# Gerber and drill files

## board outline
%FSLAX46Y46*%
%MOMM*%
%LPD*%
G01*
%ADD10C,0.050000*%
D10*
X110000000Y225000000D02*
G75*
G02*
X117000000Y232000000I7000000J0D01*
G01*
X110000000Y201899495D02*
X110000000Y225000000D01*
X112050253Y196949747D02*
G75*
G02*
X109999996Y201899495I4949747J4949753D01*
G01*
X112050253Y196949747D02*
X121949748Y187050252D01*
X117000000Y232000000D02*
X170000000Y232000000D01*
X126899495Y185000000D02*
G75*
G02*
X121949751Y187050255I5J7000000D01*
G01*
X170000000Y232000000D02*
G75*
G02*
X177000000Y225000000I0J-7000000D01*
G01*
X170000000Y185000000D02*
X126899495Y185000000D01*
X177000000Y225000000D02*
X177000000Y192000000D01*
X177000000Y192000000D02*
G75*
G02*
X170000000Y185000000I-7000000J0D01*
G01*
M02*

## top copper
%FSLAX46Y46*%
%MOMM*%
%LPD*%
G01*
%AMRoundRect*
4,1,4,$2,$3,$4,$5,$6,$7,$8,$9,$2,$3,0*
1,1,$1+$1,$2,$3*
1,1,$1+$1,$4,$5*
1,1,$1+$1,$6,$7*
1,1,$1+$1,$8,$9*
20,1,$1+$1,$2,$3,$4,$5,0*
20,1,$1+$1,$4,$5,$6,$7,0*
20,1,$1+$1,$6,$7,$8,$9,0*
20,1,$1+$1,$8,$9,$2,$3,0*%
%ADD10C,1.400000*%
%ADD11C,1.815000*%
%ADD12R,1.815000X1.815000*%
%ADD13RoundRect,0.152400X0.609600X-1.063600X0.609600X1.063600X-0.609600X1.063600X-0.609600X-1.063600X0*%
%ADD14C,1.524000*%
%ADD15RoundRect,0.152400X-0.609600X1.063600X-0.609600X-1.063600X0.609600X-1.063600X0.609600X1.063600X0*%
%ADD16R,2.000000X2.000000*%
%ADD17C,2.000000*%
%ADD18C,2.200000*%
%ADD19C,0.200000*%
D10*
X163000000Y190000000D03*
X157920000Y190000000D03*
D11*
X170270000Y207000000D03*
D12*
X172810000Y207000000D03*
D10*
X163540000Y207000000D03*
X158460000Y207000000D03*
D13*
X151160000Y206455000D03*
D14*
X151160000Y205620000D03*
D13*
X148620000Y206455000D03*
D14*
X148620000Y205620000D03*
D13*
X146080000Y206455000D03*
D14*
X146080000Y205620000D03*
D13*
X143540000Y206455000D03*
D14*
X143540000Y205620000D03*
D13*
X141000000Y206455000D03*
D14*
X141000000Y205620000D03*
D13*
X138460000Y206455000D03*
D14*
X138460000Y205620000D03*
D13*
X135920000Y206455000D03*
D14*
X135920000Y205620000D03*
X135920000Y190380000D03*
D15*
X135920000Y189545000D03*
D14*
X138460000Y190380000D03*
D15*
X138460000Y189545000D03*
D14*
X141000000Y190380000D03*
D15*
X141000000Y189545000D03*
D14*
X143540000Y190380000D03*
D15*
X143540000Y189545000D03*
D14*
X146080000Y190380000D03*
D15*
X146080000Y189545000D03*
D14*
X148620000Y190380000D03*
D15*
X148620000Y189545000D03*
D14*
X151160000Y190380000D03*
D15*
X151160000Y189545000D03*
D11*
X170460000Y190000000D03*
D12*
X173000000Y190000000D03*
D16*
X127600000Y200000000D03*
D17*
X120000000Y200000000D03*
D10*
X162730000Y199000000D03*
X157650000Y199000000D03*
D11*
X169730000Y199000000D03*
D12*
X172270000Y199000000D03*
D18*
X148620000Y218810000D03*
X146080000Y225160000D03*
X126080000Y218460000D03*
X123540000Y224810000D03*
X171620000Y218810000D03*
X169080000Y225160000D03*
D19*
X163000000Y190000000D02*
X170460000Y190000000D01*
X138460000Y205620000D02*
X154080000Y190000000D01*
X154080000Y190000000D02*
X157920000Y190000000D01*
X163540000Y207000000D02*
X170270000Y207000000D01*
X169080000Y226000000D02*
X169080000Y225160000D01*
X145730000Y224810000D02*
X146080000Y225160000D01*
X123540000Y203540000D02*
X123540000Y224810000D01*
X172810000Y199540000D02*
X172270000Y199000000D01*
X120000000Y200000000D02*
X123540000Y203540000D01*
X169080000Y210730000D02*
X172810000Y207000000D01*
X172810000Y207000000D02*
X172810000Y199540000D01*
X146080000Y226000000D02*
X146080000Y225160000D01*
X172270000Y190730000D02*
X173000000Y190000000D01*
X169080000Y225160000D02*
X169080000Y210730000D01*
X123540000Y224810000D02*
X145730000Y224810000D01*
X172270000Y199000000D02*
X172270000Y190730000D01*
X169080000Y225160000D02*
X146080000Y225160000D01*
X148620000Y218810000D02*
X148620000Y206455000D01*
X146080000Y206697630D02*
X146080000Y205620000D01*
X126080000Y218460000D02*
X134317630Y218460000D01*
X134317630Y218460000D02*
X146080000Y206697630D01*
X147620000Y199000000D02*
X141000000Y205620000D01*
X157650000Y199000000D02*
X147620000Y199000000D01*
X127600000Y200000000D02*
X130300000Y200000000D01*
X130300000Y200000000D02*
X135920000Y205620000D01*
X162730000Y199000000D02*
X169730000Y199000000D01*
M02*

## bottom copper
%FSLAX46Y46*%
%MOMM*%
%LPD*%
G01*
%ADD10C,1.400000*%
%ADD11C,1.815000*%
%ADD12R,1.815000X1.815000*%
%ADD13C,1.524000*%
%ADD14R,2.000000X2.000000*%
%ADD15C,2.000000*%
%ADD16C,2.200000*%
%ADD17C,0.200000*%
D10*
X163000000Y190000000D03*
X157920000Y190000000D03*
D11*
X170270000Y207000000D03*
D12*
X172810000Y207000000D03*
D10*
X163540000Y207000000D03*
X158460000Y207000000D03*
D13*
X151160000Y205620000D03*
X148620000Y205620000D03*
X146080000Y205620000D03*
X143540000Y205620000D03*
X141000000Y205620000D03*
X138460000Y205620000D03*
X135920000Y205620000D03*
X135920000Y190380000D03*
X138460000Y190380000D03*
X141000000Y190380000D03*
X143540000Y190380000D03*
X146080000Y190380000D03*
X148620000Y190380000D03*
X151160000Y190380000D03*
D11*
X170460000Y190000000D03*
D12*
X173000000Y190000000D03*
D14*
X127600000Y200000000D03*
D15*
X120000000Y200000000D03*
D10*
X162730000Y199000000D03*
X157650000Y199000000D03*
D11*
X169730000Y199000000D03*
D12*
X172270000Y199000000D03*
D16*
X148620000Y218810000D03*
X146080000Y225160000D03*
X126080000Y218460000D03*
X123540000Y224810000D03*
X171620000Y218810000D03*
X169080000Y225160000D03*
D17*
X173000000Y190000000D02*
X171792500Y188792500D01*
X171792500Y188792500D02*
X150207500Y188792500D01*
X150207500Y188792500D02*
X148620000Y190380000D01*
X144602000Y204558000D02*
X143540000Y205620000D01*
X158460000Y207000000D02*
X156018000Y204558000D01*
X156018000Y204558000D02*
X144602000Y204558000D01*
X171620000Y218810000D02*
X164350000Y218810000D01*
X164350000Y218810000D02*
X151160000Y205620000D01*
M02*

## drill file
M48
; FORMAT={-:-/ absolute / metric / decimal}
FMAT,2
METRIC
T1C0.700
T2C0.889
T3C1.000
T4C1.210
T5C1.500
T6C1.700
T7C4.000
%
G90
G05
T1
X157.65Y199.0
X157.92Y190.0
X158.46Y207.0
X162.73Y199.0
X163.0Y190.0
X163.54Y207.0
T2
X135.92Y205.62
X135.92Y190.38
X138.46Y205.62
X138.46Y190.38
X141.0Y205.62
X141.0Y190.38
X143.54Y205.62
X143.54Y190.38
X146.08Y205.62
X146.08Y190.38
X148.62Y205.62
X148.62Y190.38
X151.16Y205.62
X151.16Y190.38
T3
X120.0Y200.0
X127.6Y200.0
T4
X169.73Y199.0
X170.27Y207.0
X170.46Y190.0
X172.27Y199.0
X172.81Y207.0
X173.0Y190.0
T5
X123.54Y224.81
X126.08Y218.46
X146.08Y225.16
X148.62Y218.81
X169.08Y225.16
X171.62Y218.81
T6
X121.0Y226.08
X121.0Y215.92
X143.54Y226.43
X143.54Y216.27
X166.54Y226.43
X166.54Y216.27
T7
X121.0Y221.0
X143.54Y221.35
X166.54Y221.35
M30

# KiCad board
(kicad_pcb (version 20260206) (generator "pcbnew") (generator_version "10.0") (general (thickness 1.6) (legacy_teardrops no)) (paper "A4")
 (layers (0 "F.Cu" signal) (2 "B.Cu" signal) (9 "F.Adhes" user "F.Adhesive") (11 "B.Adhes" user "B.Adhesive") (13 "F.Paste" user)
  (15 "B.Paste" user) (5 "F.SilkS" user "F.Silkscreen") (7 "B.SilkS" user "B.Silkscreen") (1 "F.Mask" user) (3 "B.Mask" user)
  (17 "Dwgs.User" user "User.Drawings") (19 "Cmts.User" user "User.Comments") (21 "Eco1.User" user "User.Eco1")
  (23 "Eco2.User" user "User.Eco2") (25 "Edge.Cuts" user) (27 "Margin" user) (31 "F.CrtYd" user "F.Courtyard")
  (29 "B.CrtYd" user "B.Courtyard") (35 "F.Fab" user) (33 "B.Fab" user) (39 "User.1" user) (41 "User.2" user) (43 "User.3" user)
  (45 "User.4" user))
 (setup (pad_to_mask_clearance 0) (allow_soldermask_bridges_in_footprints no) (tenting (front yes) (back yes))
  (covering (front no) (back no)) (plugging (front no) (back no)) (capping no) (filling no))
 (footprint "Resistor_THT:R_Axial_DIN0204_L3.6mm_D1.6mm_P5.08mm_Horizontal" (layer "F.Cu") (at 163 -190 180)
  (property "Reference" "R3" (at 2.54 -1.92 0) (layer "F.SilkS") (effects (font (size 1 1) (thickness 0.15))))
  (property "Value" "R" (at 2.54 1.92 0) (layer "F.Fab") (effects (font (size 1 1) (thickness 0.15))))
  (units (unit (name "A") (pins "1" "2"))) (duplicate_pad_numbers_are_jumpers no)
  (pad "1" thru_hole circle (at 0 0 180) (size 1.4 1.4) (drill 0.7) (layers "*.Cu" "*.Mask") (remove_unused_layers no) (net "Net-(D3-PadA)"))
  (pad "2" thru_hole circle (at 5.08 0 180) (size 1.4 1.4) (drill 0.7) (layers "*.Cu" "*.Mask") (remove_unused_layers no) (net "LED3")))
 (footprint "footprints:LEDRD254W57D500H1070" (layer "F.Cu") (at 171.54 -207 180)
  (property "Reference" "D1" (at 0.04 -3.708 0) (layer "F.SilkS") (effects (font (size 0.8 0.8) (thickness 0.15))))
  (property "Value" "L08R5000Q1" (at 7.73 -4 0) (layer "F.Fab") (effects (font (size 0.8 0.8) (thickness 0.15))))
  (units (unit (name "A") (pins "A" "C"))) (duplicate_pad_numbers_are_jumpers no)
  (pad "A" thru_hole circle (at 1.27 0 180) (size 1.815 1.815) (drill 1.21) (layers "*.Cu" "*.Mask") (remove_unused_layers no)
   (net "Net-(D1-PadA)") (solder_mask_margin 0.102))
  (pad "C" thru_hole rect (at -1.27 0 180) (size 1.815 1.815) (drill 1.21) (layers "*.Cu" "*.Mask") (remove_unused_layers no) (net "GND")
   (solder_mask_margin 0.102)))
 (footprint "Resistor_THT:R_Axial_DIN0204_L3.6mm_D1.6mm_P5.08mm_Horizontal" (layer "F.Cu") (at 163.54 -207 180)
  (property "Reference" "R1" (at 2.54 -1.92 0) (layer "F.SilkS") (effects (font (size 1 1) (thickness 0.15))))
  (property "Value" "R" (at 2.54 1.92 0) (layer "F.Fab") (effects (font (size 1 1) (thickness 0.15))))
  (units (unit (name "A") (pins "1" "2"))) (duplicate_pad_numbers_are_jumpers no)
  (pad "1" thru_hole circle (at 0 0 180) (size 1.4 1.4) (drill 0.7) (layers "*.Cu" "*.Mask") (remove_unused_layers no) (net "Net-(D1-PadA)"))
  (pad "2" thru_hole circle (at 5.08 0 180) (size 1.4 1.4) (drill 0.7) (layers "*.Cu" "*.Mask") (remove_unused_layers no) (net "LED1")))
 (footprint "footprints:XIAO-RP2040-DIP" (layer "F.Cu") (at 143.54 -198)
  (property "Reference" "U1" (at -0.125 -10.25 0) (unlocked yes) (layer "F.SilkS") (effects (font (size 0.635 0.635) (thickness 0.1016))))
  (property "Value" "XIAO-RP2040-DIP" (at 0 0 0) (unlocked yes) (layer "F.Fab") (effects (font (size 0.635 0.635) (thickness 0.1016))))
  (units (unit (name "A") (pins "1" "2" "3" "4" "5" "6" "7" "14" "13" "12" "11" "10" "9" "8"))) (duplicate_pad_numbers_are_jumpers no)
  (pad "1" smd roundrect (at 7.62 -8.455 90) (size 2.432 1.524) (layers "F.Cu" "F.Mask") (roundrect_rratio 0.1) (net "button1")
   (thermal_bridge_angle 45))
  (pad "1" thru_hole circle (at 7.62 -7.62 90) (size 1.524 1.524) (drill 0.889) (layers "*.Cu" "*.Mask") (remove_unused_layers no)
   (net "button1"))
  (pad "2" smd roundrect (at 5.08 -8.455 90) (size 2.432 1.524) (layers "F.Cu" "F.Mask") (roundrect_rratio 0.1) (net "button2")
   (thermal_bridge_angle 45))
  (pad "2" thru_hole circle (at 5.08 -7.62 90) (size 1.524 1.524) (drill 0.889) (layers "*.Cu" "*.Mask") (remove_unused_layers no)
   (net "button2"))
  (pad "3" smd roundrect (at 2.54 -8.455 90) (size 2.432 1.524) (layers "F.Cu" "F.Mask") (roundrect_rratio 0.1) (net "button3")
   (thermal_bridge_angle 45))
  (pad "3" thru_hole circle (at 2.54 -7.62 90) (size 1.524 1.524) (drill 0.889) (layers "*.Cu" "*.Mask") (remove_unused_layers no)
   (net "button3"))
  (pad "4" smd roundrect (at 0 -8.455 90) (size 2.432 1.524) (layers "F.Cu" "F.Mask") (roundrect_rratio 0.1) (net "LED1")
   (thermal_bridge_angle 45))
  (pad "4" thru_hole circle (at 0 -7.62 90) (size 1.524 1.524) (drill 0.889) (layers "*.Cu" "*.Mask") (remove_unused_layers no) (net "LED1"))
  (pad "5" smd roundrect (at -2.54 -8.455 90) (size 2.432 1.524) (layers "F.Cu" "F.Mask") (roundrect_rratio 0.1) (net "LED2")
   (thermal_bridge_angle 45))
  (pad "5" thru_hole circle (at -2.54 -7.62 90) (size 1.524 1.524) (drill 0.889) (layers "*.Cu" "*.Mask") (remove_unused_layers no)
   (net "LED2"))
  (pad "6" smd roundrect (at -5.08 -8.455 90) (size 2.432 1.524) (layers "F.Cu" "F.Mask") (roundrect_rratio 0.1) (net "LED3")
   (thermal_bridge_angle 45))
  (pad "6" thru_hole circle (at -5.08 -7.62 90) (size 1.524 1.524) (drill 0.889) (layers "*.Cu" "*.Mask") (remove_unused_layers no)
   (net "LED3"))
  (pad "7" smd roundrect (at -7.62 -8.455 90) (size 2.432 1.524) (layers "F.Cu" "F.Mask") (roundrect_rratio 0.1) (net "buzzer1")
   (thermal_bridge_angle 45))
  (pad "7" thru_hole circle (at -7.62 -7.62 90) (size 1.524 1.524) (drill 0.889) (layers "*.Cu" "*.Mask") (remove_unused_layers no)
   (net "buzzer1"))
  (pad "8" thru_hole circle (at -7.62 7.62 270) (size 1.524 1.524) (drill 0.889) (layers "*.Cu" "*.Mask") (remove_unused_layers no)
   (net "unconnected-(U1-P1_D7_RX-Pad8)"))
  (pad "8" smd roundrect (at -7.62 8.455 270) (size 2.432 1.524) (layers "F.Cu" "F.Mask") (roundrect_rratio 0.1)
   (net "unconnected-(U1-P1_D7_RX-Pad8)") (thermal_bridge_angle 45))
  (pad "9" thru_hole circle (at -5.08 7.62 270) (size 1.524 1.524) (drill 0.889) (layers "*.Cu" "*.Mask") (remove_unused_layers no)
   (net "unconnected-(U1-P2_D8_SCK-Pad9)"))
  (pad "9" smd roundrect (at -5.08 8.455 270) (size 2.432 1.524) (layers "F.Cu" "F.Mask") (roundrect_rratio 0.1)
   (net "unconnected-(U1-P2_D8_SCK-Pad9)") (thermal_bridge_angle 45))
  (pad "10" thru_hole circle (at -2.54 7.62 270) (size 1.524 1.524) (drill 0.889) (layers "*.Cu" "*.Mask") (remove_unused_layers no)
   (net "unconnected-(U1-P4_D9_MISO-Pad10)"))
  (pad "10" smd roundrect (at -2.54 8.455 270) (size 2.432 1.524) (layers "F.Cu" "F.Mask") (roundrect_rratio 0.1)
   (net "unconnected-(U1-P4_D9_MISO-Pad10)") (thermal_bridge_angle 45))
  (pad "11" thru_hole circle (at 0 7.62 270) (size 1.524 1.524) (drill 0.889) (layers "*.Cu" "*.Mask") (remove_unused_layers no)
   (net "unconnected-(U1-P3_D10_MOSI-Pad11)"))
  (pad "11" smd roundrect (at 0 8.455 270) (size 2.432 1.524) (layers "F.Cu" "F.Mask") (roundrect_rratio 0.1)
   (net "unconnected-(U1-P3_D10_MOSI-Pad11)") (thermal_bridge_angle 45))
  (pad "12" thru_hole circle (at 2.54 7.62 270) (size 1.524 1.524) (drill 0.889) (layers "*.Cu" "*.Mask") (remove_unused_layers no)
   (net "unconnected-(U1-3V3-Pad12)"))
  (pad "12" smd roundrect (at 2.54 8.455 270) (size 2.432 1.524) (layers "F.Cu" "F.Mask") (roundrect_rratio 0.1)
   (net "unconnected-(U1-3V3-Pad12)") (thermal_bridge_angle 45))
  (pad "13" thru_hole circle (at 5.08 7.62 270) (size 1.524 1.524) (drill 0.889) (layers "*.Cu" "*.Mask") (remove_unused_layers no)
   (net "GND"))
  (pad "13" smd roundrect (at 5.08 8.455 270) (size 2.432 1.524) (layers "F.Cu" "F.Mask") (roundrect_rratio 0.1) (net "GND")
   (thermal_bridge_angle 45))
  (pad "14" thru_hole circle (at 7.62 7.62 270) (size 1.524 1.524) (drill 0.889) (layers "*.Cu" "*.Mask") (remove_unused_layers no)
   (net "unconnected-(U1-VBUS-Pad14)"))
  (pad "14" smd roundrect (at 7.62 8.455 270) (size 2.432 1.524) (layers "F.Cu" "F.Mask") (roundrect_rratio 0.1)
   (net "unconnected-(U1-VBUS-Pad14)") (thermal_bridge_angle 45)))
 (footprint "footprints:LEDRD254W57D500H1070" (layer "F.Cu") (at 171.73 -190 180)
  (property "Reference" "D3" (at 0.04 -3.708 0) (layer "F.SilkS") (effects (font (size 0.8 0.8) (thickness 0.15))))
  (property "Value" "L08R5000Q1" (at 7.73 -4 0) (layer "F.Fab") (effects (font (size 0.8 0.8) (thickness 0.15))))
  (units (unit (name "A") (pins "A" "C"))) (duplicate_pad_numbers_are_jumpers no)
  (pad "A" thru_hole circle (at 1.27 0 180) (size 1.815 1.815) (drill 1.21) (layers "*.Cu" "*.Mask") (remove_unused_layers no)
   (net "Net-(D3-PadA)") (solder_mask_margin 0.102))
  (pad "C" thru_hole rect (at -1.27 0 180) (size 1.815 1.815) (drill 1.21) (layers "*.Cu" "*.Mask") (remove_unused_layers no) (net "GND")
   (solder_mask_margin 0.102)))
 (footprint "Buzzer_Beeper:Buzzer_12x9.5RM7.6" (layer "F.Cu") (at 127.6 -200 180)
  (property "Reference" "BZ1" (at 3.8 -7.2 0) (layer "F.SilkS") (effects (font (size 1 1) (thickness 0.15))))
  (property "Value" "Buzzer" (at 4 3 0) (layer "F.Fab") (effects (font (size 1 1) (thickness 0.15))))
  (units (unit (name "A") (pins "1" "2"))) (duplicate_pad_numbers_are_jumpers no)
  (pad "1" thru_hole rect (at 0 0 180) (size 2 2) (drill 1) (layers "*.Cu" "*.Mask") (remove_unused_layers no) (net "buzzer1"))
  (pad "2" thru_hole circle (at 7.6 0 180) (size 2 2) (drill 1) (layers "*.Cu" "*.Mask") (remove_unused_layers no) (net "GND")))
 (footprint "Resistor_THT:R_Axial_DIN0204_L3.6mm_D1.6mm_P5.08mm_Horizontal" (layer "F.Cu") (at 162.73 -199 180)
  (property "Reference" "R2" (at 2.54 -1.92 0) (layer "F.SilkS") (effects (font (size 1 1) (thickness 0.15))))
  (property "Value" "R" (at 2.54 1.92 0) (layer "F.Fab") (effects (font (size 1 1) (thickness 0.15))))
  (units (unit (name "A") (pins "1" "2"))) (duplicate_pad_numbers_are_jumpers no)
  (pad "1" thru_hole circle (at 0 0 180) (size 1.4 1.4) (drill 0.7) (layers "*.Cu" "*.Mask") (remove_unused_layers no) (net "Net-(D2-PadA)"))
  (pad "2" thru_hole circle (at 5.08 0 180) (size 1.4 1.4) (drill 0.7) (layers "*.Cu" "*.Mask") (remove_unused_layers no) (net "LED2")))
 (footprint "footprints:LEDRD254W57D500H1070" (layer "F.Cu") (at 171 -199 180)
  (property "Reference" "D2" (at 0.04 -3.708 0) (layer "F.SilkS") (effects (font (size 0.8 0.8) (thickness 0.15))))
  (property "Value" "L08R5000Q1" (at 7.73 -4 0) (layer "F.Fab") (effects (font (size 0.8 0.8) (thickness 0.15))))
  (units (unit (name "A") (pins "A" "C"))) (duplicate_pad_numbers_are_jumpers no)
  (pad "A" thru_hole circle (at 1.27 0 180) (size 1.815 1.815) (drill 1.21) (layers "*.Cu" "*.Mask") (remove_unused_layers no)
   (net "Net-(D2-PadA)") (solder_mask_margin 0.102))
  (pad "C" thru_hole rect (at -1.27 0 180) (size 1.815 1.815) (drill 1.21) (layers "*.Cu" "*.Mask") (remove_unused_layers no) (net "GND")
   (solder_mask_margin 0.102)))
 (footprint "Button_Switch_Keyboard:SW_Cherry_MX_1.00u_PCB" (layer "F.Cu") (at 148.62 -218.81 -90)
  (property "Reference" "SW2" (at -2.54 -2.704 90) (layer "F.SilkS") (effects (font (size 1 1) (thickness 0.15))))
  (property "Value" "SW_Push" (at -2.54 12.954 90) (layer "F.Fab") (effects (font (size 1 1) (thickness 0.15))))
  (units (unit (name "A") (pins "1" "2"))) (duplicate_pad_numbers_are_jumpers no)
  (pad "" np_thru_hole circle (at -7.62 5.08 270) (size 1.7 1.7) (drill 1.7) (layers "*.Cu" "*.Mask"))
  (pad "" np_thru_hole circle (at -2.54 5.08 270) (size 4 4) (drill 4) (layers "*.Cu" "*.Mask"))
  (pad "" np_thru_hole circle (at 2.54 5.08 270) (size 1.7 1.7) (drill 1.7) (layers "*.Cu" "*.Mask"))
  (pad "1" thru_hole circle (at 0 0 270) (size 2.2 2.2) (drill 1.5) (layers "*.Cu" "*.Mask") (remove_unused_layers no) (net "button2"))
  (pad "2" thru_hole circle (at -6.35 2.54 270) (size 2.2 2.2) (drill 1.5) (layers "*.Cu" "*.Mask") (remove_unused_layers no) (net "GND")))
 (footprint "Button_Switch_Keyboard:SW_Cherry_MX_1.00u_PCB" (layer "F.Cu") (at 126.08 -218.46 -90)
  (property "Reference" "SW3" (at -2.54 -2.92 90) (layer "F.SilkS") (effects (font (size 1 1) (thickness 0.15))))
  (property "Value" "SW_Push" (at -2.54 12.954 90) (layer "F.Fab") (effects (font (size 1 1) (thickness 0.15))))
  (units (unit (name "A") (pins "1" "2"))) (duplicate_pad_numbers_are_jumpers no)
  (pad "" np_thru_hole circle (at -7.62 5.08 270) (size 1.7 1.7) (drill 1.7) (layers "*.Cu" "*.Mask"))
  (pad "" np_thru_hole circle (at -2.54 5.08 270) (size 4 4) (drill 4) (layers "*.Cu" "*.Mask"))
  (pad "" np_thru_hole circle (at 2.54 5.08 270) (size 1.7 1.7) (drill 1.7) (layers "*.Cu" "*.Mask"))
  (pad "1" thru_hole circle (at 0 0 270) (size 2.2 2.2) (drill 1.5) (layers "*.Cu" "*.Mask") (remove_unused_layers no) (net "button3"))
  (pad "2" thru_hole circle (at -6.35 2.54 270) (size 2.2 2.2) (drill 1.5) (layers "*.Cu" "*.Mask") (remove_unused_layers no) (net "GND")))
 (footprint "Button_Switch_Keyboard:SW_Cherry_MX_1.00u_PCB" (layer "F.Cu") (at 171.62 -218.81 -90)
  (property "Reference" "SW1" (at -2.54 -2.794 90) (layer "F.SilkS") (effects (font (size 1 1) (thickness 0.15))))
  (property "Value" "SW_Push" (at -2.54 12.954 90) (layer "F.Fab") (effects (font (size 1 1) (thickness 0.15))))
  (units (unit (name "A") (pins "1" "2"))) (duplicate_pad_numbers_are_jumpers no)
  (pad "" np_thru_hole circle (at -7.62 5.08 270) (size 1.7 1.7) (drill 1.7) (layers "*.Cu" "*.Mask"))
  (pad "" np_thru_hole circle (at -2.54 5.08 270) (size 4 4) (drill 4) (layers "*.Cu" "*.Mask"))
  (pad "" np_thru_hole circle (at 2.54 5.08 270) (size 1.7 1.7) (drill 1.7) (layers "*.Cu" "*.Mask"))
  (pad "1" thru_hole circle (at 0 0 270) (size 2.2 2.2) (drill 1.5) (layers "*.Cu" "*.Mask") (remove_unused_layers no) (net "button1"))
  (pad "2" thru_hole circle (at -6.35 2.54 270) (size 2.2 2.2) (drill 1.5) (layers "*.Cu" "*.Mask") (remove_unused_layers no) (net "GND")))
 (gr_arc (start 110 -225) (mid 112.050253 -229.949747) (end 117 -232) (stroke (width 0.05) (type default)) (layer "Edge.Cuts"))
 (gr_line (start 110 -201.899495) (end 110 -225) (stroke (width 0.05) (type default)) (layer "Edge.Cuts"))
 (gr_arc (start 112.050253 -196.949747) (mid 110.532842 -199.22071) (end 110 -201.899495) (stroke (width 0.05) (type default))
  (layer "Edge.Cuts"))
 (gr_line (start 112.050253 -196.949747) (end 121.949748 -187.050252) (stroke (width 0.05) (type default)) (layer "Edge.Cuts"))
 (gr_line (start 117 -232) (end 170 -232) (stroke (width 0.05) (type default)) (layer "Edge.Cuts"))
 (gr_arc (start 126.899495 -185) (mid 124.220711 -185.532843) (end 121.949748 -187.050252) (stroke (width 0.05) (type default))
  (layer "Edge.Cuts"))
 (gr_arc (start 170 -232) (mid 174.949747 -229.949747) (end 177 -225) (stroke (width 0.05) (type default)) (layer "Edge.Cuts"))
 (gr_line (start 170 -185) (end 126.899495 -185) (stroke (width 0.05) (type default)) (layer "Edge.Cuts"))
 (gr_line (start 177 -225) (end 177 -192) (stroke (width 0.05) (type default)) (layer "Edge.Cuts"))
 (gr_arc (start 177 -192) (mid 174.949747 -187.050253) (end 170 -185) (stroke (width 0.05) (type default)) (layer "Edge.Cuts"))
 (segment (start 163 -190) (end 170.46 -190) (width 0.2) (layer "F.Cu") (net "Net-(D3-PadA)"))
 (segment (start 138.46 -205.62) (end 154.08 -190) (width 0.2) (layer "F.Cu") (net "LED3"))
 (segment (start 154.08 -190) (end 157.92 -190) (width 0.2) (layer "F.Cu") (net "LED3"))
 (segment (start 163.54 -207) (end 170.27 -207) (width 0.2) (layer "F.Cu") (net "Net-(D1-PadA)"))
 (segment (start 169.08 -226) (end 169.08 -225.16) (width 0.2) (layer "F.Cu") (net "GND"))
 (segment (start 145.73 -224.81) (end 146.08 -225.16) (width 0.2) (layer "F.Cu") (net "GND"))
 (segment (start 123.54 -203.54) (end 123.54 -224.81) (width 0.2) (layer "F.Cu") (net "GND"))
 (segment (start 172.81 -199.54) (end 172.27 -199) (width 0.2) (layer "F.Cu") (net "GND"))
 (segment (start 120 -200) (end 123.54 -203.54) (width 0.2) (layer "F.Cu") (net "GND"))
 (segment (start 169.08 -210.73) (end 172.81 -207) (width 0.2) (layer "F.Cu") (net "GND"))
 (segment (start 172.81 -207) (end 172.81 -199.54) (width 0.2) (layer "F.Cu") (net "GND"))
 (segment (start 146.08 -226) (end 146.08 -225.16) (width 0.2) (layer "F.Cu") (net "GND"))
 (segment (start 172.27 -190.73) (end 173 -190) (width 0.2) (layer "F.Cu") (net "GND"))
 (segment (start 169.08 -225.16) (end 169.08 -210.73) (width 0.2) (layer "F.Cu") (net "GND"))
 (segment (start 123.54 -224.81) (end 145.73 -224.81) (width 0.2) (layer "F.Cu") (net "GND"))
 (segment (start 172.27 -199) (end 172.27 -190.73) (width 0.2) (layer "F.Cu") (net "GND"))
 (segment (start 169.08 -225.16) (end 146.08 -225.16) (width 0.2) (layer "F.Cu") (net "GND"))
 (segment (start 173 -190) (end 171.7925 -188.7925) (width 0.2) (layer "B.Cu") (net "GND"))
 (segment (start 171.7925 -188.7925) (end 150.2075 -188.7925) (width 0.2) (layer "B.Cu") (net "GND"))
 (segment (start 150.2075 -188.7925) (end 148.62 -190.38) (width 0.2) (layer "B.Cu") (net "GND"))
 (segment (start 144.602 -204.558) (end 143.54 -205.62) (width 0.2) (layer "B.Cu") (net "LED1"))
 (segment (start 158.46 -207) (end 156.018 -204.558) (width 0.2) (layer "B.Cu") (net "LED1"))
 (segment (start 156.018 -204.558) (end 144.602 -204.558) (width 0.2) (layer "B.Cu") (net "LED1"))
 (segment (start 171.62 -218.81) (end 164.35 -218.81) (width 0.2) (layer "B.Cu") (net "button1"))
 (segment (start 164.35 -218.81) (end 151.16 -205.62) (width 0.2) (layer "B.Cu") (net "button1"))
 (segment (start 148.62 -218.81) (end 148.62 -206.455) (width 0.2) (layer "F.Cu") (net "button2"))
 (segment (start 146.08 -206.69763) (end 146.08 -205.62) (width 0.2) (layer "F.Cu") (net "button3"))
 (segment (start 126.08 -218.46) (end 134.31763 -218.46) (width 0.2) (layer "F.Cu") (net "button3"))
 (segment (start 134.31763 -218.46) (end 146.08 -206.69763) (width 0.2) (layer "F.Cu") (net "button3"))
 (segment (start 147.62 -199) (end 141 -205.62) (width 0.2) (layer "F.Cu") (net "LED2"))
 (segment (start 157.65 -199) (end 147.62 -199) (width 0.2) (layer "F.Cu") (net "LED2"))
 (segment (start 127.6 -200) (end 130.3 -200) (width 0.2) (layer "F.Cu") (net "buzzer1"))
 (segment (start 130.3 -200) (end 135.92 -205.62) (width 0.2) (layer "F.Cu") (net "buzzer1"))
 (segment (start 162.73 -199) (end 169.73 -199) (width 0.2) (layer "F.Cu") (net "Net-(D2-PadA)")))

